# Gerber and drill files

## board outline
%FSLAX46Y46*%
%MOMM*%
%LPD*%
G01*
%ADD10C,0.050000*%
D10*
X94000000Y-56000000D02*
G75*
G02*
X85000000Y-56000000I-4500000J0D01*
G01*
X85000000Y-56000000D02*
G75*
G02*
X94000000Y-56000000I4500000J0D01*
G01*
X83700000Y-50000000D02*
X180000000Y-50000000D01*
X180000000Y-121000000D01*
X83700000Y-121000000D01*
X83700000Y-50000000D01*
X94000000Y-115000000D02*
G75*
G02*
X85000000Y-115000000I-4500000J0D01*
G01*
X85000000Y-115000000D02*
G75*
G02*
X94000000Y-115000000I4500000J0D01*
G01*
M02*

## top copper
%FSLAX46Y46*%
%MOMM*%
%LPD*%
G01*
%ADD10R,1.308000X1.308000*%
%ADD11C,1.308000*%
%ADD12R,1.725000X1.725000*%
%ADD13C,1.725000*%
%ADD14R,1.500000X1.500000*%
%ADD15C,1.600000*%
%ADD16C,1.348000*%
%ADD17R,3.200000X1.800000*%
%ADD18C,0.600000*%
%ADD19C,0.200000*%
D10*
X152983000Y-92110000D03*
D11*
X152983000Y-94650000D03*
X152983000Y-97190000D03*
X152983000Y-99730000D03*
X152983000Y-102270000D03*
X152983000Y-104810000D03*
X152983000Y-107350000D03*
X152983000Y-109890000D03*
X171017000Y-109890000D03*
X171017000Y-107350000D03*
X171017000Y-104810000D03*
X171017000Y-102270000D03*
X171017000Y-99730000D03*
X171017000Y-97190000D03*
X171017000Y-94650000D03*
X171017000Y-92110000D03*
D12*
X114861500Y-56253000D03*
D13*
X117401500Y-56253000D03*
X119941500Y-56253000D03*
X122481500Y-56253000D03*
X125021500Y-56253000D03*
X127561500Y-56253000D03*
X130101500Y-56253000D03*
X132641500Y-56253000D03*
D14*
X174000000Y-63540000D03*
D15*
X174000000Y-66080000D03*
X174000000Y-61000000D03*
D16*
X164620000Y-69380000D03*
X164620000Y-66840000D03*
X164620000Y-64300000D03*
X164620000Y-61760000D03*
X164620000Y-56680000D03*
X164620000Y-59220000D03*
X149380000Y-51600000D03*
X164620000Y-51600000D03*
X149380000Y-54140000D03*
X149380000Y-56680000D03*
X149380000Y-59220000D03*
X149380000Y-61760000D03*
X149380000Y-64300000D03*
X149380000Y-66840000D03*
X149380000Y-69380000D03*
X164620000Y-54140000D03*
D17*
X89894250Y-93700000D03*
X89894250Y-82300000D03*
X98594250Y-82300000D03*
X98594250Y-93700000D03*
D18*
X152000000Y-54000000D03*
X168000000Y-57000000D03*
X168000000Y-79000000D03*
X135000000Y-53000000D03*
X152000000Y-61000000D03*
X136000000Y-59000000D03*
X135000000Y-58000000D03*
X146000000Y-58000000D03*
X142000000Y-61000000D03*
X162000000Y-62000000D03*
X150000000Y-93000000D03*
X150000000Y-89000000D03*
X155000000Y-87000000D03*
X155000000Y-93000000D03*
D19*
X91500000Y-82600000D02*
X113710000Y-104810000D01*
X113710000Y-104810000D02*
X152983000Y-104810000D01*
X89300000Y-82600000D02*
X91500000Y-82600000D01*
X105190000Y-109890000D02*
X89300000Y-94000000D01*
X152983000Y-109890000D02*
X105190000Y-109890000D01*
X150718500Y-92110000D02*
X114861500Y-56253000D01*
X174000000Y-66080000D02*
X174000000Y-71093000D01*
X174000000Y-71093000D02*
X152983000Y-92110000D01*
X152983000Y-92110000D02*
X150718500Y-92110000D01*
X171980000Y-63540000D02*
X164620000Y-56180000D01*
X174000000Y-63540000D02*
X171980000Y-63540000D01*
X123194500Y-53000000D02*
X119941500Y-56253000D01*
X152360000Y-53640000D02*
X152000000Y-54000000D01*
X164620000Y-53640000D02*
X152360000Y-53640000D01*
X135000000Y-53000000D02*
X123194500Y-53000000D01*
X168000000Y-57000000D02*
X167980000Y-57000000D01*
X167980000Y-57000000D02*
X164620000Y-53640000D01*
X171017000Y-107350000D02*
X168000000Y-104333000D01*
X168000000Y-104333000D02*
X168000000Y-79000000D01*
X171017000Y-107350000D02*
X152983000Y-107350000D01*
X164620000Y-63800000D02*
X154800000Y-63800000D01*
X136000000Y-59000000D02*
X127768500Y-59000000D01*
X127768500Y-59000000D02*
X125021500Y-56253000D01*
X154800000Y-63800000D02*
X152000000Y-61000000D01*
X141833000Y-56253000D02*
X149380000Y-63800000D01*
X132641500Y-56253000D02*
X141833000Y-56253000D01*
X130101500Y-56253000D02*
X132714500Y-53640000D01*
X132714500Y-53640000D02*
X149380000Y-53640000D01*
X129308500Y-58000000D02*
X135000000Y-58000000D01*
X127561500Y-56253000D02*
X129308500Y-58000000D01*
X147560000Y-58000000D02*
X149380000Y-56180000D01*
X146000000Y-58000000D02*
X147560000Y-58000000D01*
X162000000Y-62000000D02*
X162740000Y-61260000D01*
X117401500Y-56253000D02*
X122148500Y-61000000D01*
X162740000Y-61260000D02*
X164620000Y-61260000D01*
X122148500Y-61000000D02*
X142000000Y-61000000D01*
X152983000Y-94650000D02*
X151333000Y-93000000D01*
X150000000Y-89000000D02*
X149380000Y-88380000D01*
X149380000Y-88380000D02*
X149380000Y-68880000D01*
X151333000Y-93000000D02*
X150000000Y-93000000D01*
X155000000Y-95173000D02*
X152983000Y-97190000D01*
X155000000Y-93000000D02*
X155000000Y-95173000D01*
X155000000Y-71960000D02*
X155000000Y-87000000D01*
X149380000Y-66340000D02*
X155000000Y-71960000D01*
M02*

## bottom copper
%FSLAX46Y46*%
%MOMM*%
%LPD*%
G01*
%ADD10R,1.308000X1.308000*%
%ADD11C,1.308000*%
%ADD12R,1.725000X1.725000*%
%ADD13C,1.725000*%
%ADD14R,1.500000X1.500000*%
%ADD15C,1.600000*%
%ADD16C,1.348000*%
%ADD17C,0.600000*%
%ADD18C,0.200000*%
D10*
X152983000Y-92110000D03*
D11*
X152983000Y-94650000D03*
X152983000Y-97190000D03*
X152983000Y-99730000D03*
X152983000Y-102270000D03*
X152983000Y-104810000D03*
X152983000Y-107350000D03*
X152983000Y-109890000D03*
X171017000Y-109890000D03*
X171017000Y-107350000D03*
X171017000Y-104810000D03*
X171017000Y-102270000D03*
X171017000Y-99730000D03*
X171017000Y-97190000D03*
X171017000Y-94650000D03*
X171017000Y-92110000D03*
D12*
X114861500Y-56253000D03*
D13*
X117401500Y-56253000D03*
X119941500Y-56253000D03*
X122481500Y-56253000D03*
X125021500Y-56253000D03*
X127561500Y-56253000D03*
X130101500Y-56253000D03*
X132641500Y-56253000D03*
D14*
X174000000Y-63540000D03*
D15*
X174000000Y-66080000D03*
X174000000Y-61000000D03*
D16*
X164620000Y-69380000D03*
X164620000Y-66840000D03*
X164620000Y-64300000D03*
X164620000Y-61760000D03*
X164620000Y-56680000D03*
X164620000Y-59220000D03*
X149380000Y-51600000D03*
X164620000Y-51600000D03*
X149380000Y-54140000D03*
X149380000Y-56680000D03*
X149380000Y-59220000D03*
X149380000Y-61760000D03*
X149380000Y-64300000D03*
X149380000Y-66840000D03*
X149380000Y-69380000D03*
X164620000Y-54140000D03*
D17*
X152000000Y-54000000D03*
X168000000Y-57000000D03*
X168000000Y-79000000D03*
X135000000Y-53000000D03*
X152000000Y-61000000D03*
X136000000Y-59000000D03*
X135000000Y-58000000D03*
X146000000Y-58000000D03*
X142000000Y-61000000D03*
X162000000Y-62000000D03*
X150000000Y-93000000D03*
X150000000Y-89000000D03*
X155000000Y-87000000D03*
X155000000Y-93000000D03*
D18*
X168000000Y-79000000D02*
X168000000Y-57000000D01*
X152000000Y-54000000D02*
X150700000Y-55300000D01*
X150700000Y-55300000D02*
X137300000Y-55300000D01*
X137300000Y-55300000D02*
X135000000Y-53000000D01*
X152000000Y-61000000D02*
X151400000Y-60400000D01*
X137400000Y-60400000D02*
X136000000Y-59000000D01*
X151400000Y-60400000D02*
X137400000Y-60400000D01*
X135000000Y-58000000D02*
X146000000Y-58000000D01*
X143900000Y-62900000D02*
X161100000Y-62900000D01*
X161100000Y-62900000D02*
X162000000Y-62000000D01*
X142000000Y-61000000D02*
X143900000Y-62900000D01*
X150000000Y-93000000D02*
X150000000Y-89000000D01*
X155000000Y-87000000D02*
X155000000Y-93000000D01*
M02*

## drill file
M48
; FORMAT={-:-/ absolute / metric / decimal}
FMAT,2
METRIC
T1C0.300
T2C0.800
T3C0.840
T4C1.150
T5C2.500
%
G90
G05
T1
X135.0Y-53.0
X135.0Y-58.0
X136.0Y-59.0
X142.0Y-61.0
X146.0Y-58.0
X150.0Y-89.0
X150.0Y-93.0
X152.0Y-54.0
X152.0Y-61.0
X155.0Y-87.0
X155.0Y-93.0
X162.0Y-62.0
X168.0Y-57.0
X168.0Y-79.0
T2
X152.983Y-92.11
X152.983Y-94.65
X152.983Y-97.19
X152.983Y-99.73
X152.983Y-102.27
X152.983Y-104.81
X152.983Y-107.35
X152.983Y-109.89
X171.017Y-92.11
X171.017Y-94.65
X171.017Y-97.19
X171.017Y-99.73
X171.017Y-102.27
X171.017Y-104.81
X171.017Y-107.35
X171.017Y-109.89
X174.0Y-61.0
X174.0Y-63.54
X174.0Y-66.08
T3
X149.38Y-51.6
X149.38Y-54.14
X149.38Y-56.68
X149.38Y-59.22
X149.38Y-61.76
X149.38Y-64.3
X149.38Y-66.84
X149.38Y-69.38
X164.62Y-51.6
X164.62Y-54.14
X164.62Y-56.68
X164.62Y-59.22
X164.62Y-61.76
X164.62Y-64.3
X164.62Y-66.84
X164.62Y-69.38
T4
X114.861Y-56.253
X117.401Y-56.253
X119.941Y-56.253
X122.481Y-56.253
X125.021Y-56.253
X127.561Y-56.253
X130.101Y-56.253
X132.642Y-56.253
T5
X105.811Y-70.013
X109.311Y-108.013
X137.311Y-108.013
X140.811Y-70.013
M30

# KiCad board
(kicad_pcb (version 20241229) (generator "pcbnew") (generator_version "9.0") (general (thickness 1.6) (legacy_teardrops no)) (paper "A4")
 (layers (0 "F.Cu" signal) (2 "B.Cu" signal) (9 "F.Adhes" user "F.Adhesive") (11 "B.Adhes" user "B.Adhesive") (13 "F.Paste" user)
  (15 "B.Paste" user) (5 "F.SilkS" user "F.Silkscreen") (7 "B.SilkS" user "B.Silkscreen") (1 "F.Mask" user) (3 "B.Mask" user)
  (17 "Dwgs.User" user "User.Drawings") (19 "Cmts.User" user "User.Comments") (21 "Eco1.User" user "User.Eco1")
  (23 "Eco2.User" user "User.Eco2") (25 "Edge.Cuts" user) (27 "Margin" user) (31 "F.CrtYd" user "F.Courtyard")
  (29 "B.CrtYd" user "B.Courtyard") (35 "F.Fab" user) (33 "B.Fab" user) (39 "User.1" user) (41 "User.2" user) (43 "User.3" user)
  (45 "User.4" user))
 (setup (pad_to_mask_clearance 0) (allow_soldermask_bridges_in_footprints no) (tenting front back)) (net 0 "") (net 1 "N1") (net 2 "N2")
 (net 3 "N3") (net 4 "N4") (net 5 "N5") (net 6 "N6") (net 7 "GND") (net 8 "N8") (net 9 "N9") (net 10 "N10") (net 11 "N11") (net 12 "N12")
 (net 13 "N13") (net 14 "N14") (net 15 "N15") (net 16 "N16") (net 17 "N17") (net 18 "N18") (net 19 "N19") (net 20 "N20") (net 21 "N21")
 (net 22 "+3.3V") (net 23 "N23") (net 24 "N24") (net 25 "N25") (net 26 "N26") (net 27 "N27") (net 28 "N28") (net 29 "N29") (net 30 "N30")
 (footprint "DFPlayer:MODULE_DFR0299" (layer "F.Cu") (at 162 101)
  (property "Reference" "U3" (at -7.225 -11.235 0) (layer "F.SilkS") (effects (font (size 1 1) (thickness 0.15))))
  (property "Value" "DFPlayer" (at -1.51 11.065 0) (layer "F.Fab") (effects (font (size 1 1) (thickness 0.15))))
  (pad "1" thru_hole rect (at -9.017 -8.89) (size 1.308 1.308) (drill 0.8) (layers "*.Cu" "*.Mask") (remove_unused_layers no) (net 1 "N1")
   (solder_mask_margin 0.102))
  (pad "2" thru_hole circle (at -9.017 -6.35) (size 1.308 1.308) (drill 0.8) (layers "*.Cu" "*.Mask") (remove_unused_layers no) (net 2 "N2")
   (solder_mask_margin 0.102))
  (pad "3" thru_hole circle (at -9.017 -3.81) (size 1.308 1.308) (drill 0.8) (layers "*.Cu" "*.Mask") (remove_unused_layers no) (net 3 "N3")
   (solder_mask_margin 0.102))
  (pad "4" thru_hole circle (at -9.017 -1.27) (size 1.308 1.308) (drill 0.8) (layers "*.Cu" "*.Mask") (remove_unused_layers no) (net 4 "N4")
   (solder_mask_margin 0.102))
  (pad "5" thru_hole circle (at -9.017 1.27) (size 1.308 1.308) (drill 0.8) (layers "*.Cu" "*.Mask") (remove_unused_layers no) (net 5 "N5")
   (solder_mask_margin 0.102))
  (pad "6" thru_hole circle (at -9.017 3.81) (size 1.308 1.308) (drill 0.8) (layers "*.Cu" "*.Mask") (remove_unused_layers no) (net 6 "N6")
   (solder_mask_margin 0.102))
  (pad "7" thru_hole circle (at -9.017 6.35) (size 1.308 1.308) (drill 0.8) (layers "*.Cu" "*.Mask") (remove_unused_layers no) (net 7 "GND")
   (solder_mask_margin 0.102))
  (pad "8" thru_hole circle (at -9.017 8.89) (size 1.308 1.308) (drill 0.8) (layers "*.Cu" "*.Mask") (remove_unused_layers no) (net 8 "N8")
   (solder_mask_margin 0.102))
  (pad "9" thru_hole circle (at 9.017 8.89) (size 1.308 1.308) (drill 0.8) (layers "*.Cu" "*.Mask") (remove_unused_layers no) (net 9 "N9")
   (solder_mask_margin 0.102))
  (pad "10" thru_hole circle (at 9.017 6.35) (size 1.308 1.308) (drill 0.8) (layers "*.Cu" "*.Mask") (remove_unused_layers no) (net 7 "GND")
   (solder_mask_margin 0.102))
  (pad "11" thru_hole circle (at 9.017 3.81) (size 1.308 1.308) (drill 0.8) (layers "*.Cu" "*.Mask") (remove_unused_layers no)
   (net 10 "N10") (solder_mask_margin 0.102))
  (pad "12" thru_hole circle (at 9.017 1.27) (size 1.308 1.308) (drill 0.8) (layers "*.Cu" "*.Mask") (remove_unused_layers no)
   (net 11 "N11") (solder_mask_margin 0.102))
  (pad "13" thru_hole circle (at 9.017 -1.27) (size 1.308 1.308) (drill 0.8) (layers "*.Cu" "*.Mask") (remove_unused_layers no)
   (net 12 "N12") (solder_mask_margin 0.102))
  (pad "14" thru_hole circle (at 9.017 -3.81) (size 1.308 1.308) (drill 0.8) (layers "*.Cu" "*.Mask") (remove_unused_layers no)
   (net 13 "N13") (solder_mask_margin 0.102))
  (pad "15" thru_hole circle (at 9.017 -6.35) (size 1.308 1.308) (drill 0.8) (layers "*.Cu" "*.Mask") (remove_unused_layers no)
   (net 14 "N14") (solder_mask_margin 0.102))
  (pad "16" thru_hole circle (at 9.017 -8.89) (size 1.308 1.308) (drill 0.8) (layers "*.Cu" "*.Mask") (remove_unused_layers no)
   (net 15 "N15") (solder_mask_margin 0.102)))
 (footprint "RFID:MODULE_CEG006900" (layer "F.Cu") (at 123.3115 84.013)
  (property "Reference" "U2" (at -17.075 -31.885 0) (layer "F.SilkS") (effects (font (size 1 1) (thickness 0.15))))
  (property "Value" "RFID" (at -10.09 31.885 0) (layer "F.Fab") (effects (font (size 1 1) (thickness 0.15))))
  (pad "" np_thru_hole circle (at -17.5 -14) (size 2.5 2.5) (drill 2.5) (layers "*.Cu" "*.Mask"))
  (pad "" np_thru_hole circle (at -14 24) (size 2.5 2.5) (drill 2.5) (layers "*.Cu" "*.Mask"))
  (pad "" np_thru_hole circle (at 14 24) (size 2.5 2.5) (drill 2.5) (layers "*.Cu" "*.Mask"))
  (pad "" np_thru_hole circle (at 17.5 -14) (size 2.5 2.5) (drill 2.5) (layers "*.Cu" "*.Mask"))
  (pad "1" thru_hole rect (at -8.45 -27.76) (size 1.725 1.725) (drill 1.15) (layers "*.Cu" "*.Mask") (remove_unused_layers no) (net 1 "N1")
   (solder_mask_margin 0.102))
  (pad "2" thru_hole circle (at -5.91 -27.76) (size 1.725 1.725) (drill 1.15) (layers "*.Cu" "*.Mask") (remove_unused_layers no)
   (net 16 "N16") (solder_mask_margin 0.102))
  (pad "3" thru_hole circle (at -3.37 -27.76) (size 1.725 1.725) (drill 1.15) (layers "*.Cu" "*.Mask") (remove_unused_layers no)
   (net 7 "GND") (solder_mask_margin 0.102))
  (pad "4" thru_hole circle (at -0.83 -27.76) (size 1.725 1.725) (drill 1.15) (layers "*.Cu" "*.Mask") (remove_unused_layers no)
   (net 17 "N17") (solder_mask_margin 0.102))
  (pad "5" thru_hole circle (at 1.71 -27.76) (size 1.725 1.725) (drill 1.15) (layers "*.Cu" "*.Mask") (remove_unused_layers no)
   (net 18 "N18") (solder_mask_margin 0.102))
  (pad "6" thru_hole circle (at 4.25 -27.76) (size 1.725 1.725) (drill 1.15) (layers "*.Cu" "*.Mask") (remove_unused_layers no)
   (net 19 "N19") (solder_mask_margin 0.102))
  (pad "7" thru_hole circle (at 6.79 -27.76) (size 1.725 1.725) (drill 1.15) (layers "*.Cu" "*.Mask") (remove_unused_layers no)
   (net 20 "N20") (solder_mask_margin 0.102))
  (pad "8" thru_hole circle (at 9.33 -27.76) (size 1.725 1.725) (drill 1.15) (layers "*.Cu" "*.Mask") (remove_unused_layers no)
   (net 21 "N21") (solder_mask_margin 0.102)))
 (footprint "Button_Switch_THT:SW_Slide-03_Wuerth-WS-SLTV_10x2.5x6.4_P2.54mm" (layer "F.Cu") (at 174 63.54 90)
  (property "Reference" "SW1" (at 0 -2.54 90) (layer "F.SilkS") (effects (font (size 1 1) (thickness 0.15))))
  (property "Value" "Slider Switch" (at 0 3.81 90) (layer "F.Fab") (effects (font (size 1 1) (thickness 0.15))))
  (pad "1" thru_hole rect (at 0 0 90) (size 1.5 1.5) (drill 0.8) (layers "*.Cu" "*.Mask") (remove_unused_layers no) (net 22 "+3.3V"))
  (pad "2" thru_hole circle (at -2.54 0 90) (size 1.6 1.6) (drill 0.8) (layers "*.Cu" "*.Mask") (remove_unused_layers no) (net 1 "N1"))
  (pad "3" thru_hole circle (at 2.54 0 90) (size 1.6 1.6) (drill 0.8) (layers "*.Cu" "*.Mask") (remove_unused_layers no) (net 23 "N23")))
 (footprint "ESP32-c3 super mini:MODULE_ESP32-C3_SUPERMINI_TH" (layer "F.Cu") (at 157 61.5)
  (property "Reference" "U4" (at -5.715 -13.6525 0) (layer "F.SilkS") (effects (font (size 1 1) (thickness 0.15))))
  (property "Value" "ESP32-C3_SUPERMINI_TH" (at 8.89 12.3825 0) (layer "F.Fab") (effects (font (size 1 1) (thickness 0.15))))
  (pad "0" thru_hole circle (at 7.62 7.88) (size 1.348 1.348) (drill 0.84) (layers "*.Cu" "*.Mask") (remove_unused_layers no) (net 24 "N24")
   (solder_mask_margin 0.102))
  (pad "1" thru_hole circle (at 7.62 5.34) (size 1.348 1.348) (drill 0.84) (layers "*.Cu" "*.Mask") (remove_unused_layers no) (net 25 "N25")
   (solder_mask_margin 0.102))
  (pad "2" thru_hole circle (at 7.62 2.8) (size 1.348 1.348) (drill 0.84) (layers "*.Cu" "*.Mask") (remove_unused_layers no) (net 18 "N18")
   (solder_mask_margin 0.102))
  (pad "3" thru_hole circle (at 7.62 0.26) (size 1.348 1.348) (drill 0.84) (layers "*.Cu" "*.Mask") (remove_unused_layers no) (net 16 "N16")
   (solder_mask_margin 0.102))
  (pad "3.3" thru_hole circle (at 7.62 -4.82) (size 1.348 1.348) (drill 0.84) (layers "*.Cu" "*.Mask") (remove_unused_layers no)
   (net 22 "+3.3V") (solder_mask_margin 0.102))
  (pad "4" thru_hole circle (at 7.62 -2.28) (size 1.348 1.348) (drill 0.84) (layers "*.Cu" "*.Mask") (remove_unused_layers no)
   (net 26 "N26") (solder_mask_margin 0.102))
  (pad "5" thru_hole circle (at -7.62 -9.9) (size 1.348 1.348) (drill 0.84) (layers "*.Cu" "*.Mask") (remove_unused_layers no)
   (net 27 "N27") (solder_mask_margin 0.102))
  (pad "5V" thru_hole circle (at 7.62 -9.9) (size 1.348 1.348) (drill 0.84) (layers "*.Cu" "*.Mask") (remove_unused_layers no)
   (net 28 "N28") (solder_mask_margin 0.102))
  (pad "6" thru_hole circle (at -7.62 -7.36) (size 1.348 1.348) (drill 0.84) (layers "*.Cu" "*.Mask") (remove_unused_layers no)
   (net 20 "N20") (solder_mask_margin 0.102))
  (pad "7" thru_hole circle (at -7.62 -4.82) (size 1.348 1.348) (drill 0.84) (layers "*.Cu" "*.Mask") (remove_unused_layers no)
   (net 19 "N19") (solder_mask_margin 0.102))
  (pad "8" thru_hole circle (at -7.62 -2.28) (size 1.348 1.348) (drill 0.84) (layers "*.Cu" "*.Mask") (remove_unused_layers no)
   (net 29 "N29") (solder_mask_margin 0.102))
  (pad "9" thru_hole circle (at -7.62 0.26) (size 1.348 1.348) (drill 0.84) (layers "*.Cu" "*.Mask") (remove_unused_layers no)
   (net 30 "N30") (solder_mask_margin 0.102))
  (pad "10" thru_hole circle (at -7.62 2.8) (size 1.348 1.348) (drill 0.84) (layers "*.Cu" "*.Mask") (remove_unused_layers no)
   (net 21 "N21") (solder_mask_margin 0.102))
  (pad "20" thru_hole circle (at -7.62 5.34) (size 1.348 1.348) (drill 0.84) (layers "*.Cu" "*.Mask") (remove_unused_layers no) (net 3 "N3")
   (solder_mask_margin 0.102))
  (pad "21" thru_hole circle (at -7.62 7.88) (size 1.348 1.348) (drill 0.84) (layers "*.Cu" "*.Mask") (remove_unused_layers no) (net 2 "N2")
   (solder_mask_margin 0.102))
  (pad "G" thru_hole circle (at 7.62 -7.36) (size 1.348 1.348) (drill 0.84) (layers "*.Cu" "*.Mask") (remove_unused_layers no) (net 7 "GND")
   (solder_mask_margin 0.102)))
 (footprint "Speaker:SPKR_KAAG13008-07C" (layer "F.Cu") (at 94.24425 88)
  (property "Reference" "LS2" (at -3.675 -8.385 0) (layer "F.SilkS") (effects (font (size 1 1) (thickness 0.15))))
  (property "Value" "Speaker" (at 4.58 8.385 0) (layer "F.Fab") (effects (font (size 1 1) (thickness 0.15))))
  (pad "N" smd rect (at -4.35 5.7) (size 3.2 1.8) (layers "F.Cu" "F.Mask" "F.Paste") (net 8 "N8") (solder_mask_margin 0.102))
  (pad "P" smd rect (at -4.35 -5.7) (size 3.2 1.8) (layers "F.Cu" "F.Mask" "F.Paste") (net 6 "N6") (solder_mask_margin 0.102))
  (pad "S1" smd rect (at 4.35 -5.7) (size 3.2 1.8) (layers "F.Cu" "F.Mask" "F.Paste") (solder_mask_margin 0.102))
  (pad "S2" smd rect (at 4.35 5.7) (size 3.2 1.8) (layers "F.Cu" "F.Mask" "F.Paste") (solder_mask_margin 0.102)))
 (gr_circle (center 89.5 56) (end 89.5 51.5) (stroke (width 0.05) (type default)) (fill no) (layer "Edge.Cuts"))
 (gr_rect (start 83.7 50) (end 180 121) (stroke (width 0.05) (type default)) (fill no) (layer "Edge.Cuts"))
 (gr_circle (center 89.5 115) (end 89.5 110.5) (stroke (width 0.05) (type default)) (fill no) (layer "Edge.Cuts"))
 (segment (start 91.5 82.6) (end 113.71 104.81) (width 0.2) (layer "F.Cu") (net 6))
 (segment (start 113.71 104.81) (end 152.983 104.81) (width 0.2) (layer "F.Cu") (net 6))
 (segment (start 89.3 82.6) (end 91.5 82.6) (width 0.2) (layer "F.Cu") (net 6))
 (segment (start 105.19 109.89) (end 89.3 94) (width 0.2) (layer "F.Cu") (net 8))
 (segment (start 152.983 109.89) (end 105.19 109.89) (width 0.2) (layer "F.Cu") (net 8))
 (segment (start 150.7185 92.11) (end 114.8615 56.253) (width 0.2) (layer "F.Cu") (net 1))
 (segment (start 174 66.08) (end 174 71.093) (width 0.2) (layer "F.Cu") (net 1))
 (segment (start 174 71.093) (end 152.983 92.11) (width 0.2) (layer "F.Cu") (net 1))
 (segment (start 152.983 92.11) (end 150.7185 92.11) (width 0.2) (layer "F.Cu") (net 1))
 (segment (start 171.98 63.54) (end 164.62 56.18) (width 0.2) (layer "F.Cu") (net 22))
 (segment (start 174 63.54) (end 171.98 63.54) (width 0.2) (layer "F.Cu") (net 22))
 (segment (start 123.1945 53) (end 119.9415 56.253) (width 0.2) (layer "F.Cu") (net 7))
 (segment (start 152.36 53.64) (end 152 54) (width 0.2) (layer "F.Cu") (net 7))
 (segment (start 164.62 53.64) (end 152.36 53.64) (width 0.2) (layer "F.Cu") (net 7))
 (segment (start 135 53) (end 123.1945 53) (width 0.2) (layer "F.Cu") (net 7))
 (segment (start 168 57) (end 167.98 57) (width 0.2) (layer "F.Cu") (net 7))
 (segment (start 167.98 57) (end 164.62 53.64) (width 0.2) (layer "F.Cu") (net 7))
 (segment (start 171.017 107.35) (end 168 104.333) (width 0.2) (layer "F.Cu") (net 7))
 (segment (start 168 104.333) (end 168 79) (width 0.2) (layer "F.Cu") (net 7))
 (segment (start 171.017 107.35) (end 152.983 107.35) (width 0.2) (layer "F.Cu") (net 7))
 (via (at 152 54) (size 0.6) (drill 0.3) (layers "F.Cu" "B.Cu") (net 7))
 (via (at 168 57) (size 0.6) (drill 0.3) (layers "F.Cu" "B.Cu") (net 7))
 (via (at 168 79) (size 0.6) (drill 0.3) (layers "F.Cu" "B.Cu") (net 7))
 (via (at 135 53) (size 0.6) (drill 0.3) (layers "F.Cu" "B.Cu") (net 7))
 (segment (start 168 79) (end 168 57) (width 0.2) (layer "B.Cu") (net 7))
 (segment (start 152 54) (end 150.7 55.3) (width 0.2) (layer "B.Cu") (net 7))
 (segment (start 150.7 55.3) (end 137.3 55.3) (width 0.2) (layer "B.Cu") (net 7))
 (segment (start 137.3 55.3) (end 135 53) (width 0.2) (layer "B.Cu") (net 7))
 (segment (start 164.62 63.8) (end 154.8 63.8) (width 0.2) (layer "F.Cu") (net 18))
 (segment (start 136 59) (end 127.7685 59) (width 0.2) (layer "F.Cu") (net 18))
 (segment (start 127.7685 59) (end 125.0215 56.253) (width 0.2) (layer "F.Cu") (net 18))
 (segment (start 154.8 63.8) (end 152 61) (width 0.2) (layer "F.Cu") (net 18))
 (via (at 152 61) (size 0.6) (drill 0.3) (layers "F.Cu" "B.Cu") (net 18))
 (via (at 136 59) (size 0.6) (drill 0.3) (layers "F.Cu" "B.Cu") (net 18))
 (segment (start 152 61) (end 151.4 60.4) (width 0.2) (layer "B.Cu") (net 18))
 (segment (start 137.4 60.4) (end 136 59) (width 0.2) (layer "B.Cu") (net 18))
 (segment (start 151.4 60.4) (end 137.4 60.4) (width 0.2) (layer "B.Cu") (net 18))
 (segment (start 141.833 56.253) (end 149.38 63.8) (width 0.2) (layer "F.Cu") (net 21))
 (segment (start 132.6415 56.253) (end 141.833 56.253) (width 0.2) (layer "F.Cu") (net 21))
 (segment (start 130.1015 56.253) (end 132.7145 53.64) (width 0.2) (layer "F.Cu") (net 20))
 (segment (start 132.7145 53.64) (end 149.38 53.64) (width 0.2) (layer "F.Cu") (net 20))
 (segment (start 129.3085 58) (end 135 58) (width 0.2) (layer "F.Cu") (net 19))
 (segment (start 127.5615 56.253) (end 129.3085 58) (width 0.2) (layer "F.Cu") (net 19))
 (segment (start 147.56 58) (end 149.38 56.18) (width 0.2) (layer "F.Cu") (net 19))
 (segment (start 146 58) (end 147.56 58) (width 0.2) (layer "F.Cu") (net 19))
 (via (at 135 58) (size 0.6) (drill 0.3) (layers "F.Cu" "B.Cu") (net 19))
 (via (at 146 58) (size 0.6) (drill 0.3) (layers "F.Cu" "B.Cu") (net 19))
 (segment (start 135 58) (end 146 58) (width 0.2) (layer "B.Cu") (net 19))
 (segment (start 162 62) (end 162.74 61.26) (width 0.2) (layer "F.Cu") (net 16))
 (segment (start 117.4015 56.253) (end 122.1485 61) (width 0.2) (layer "F.Cu") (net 16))
 (segment (start 162.74 61.26) (end 164.62 61.26) (width 0.2) (layer "F.Cu") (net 16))
 (segment (start 122.1485 61) (end 142 61) (width 0.2) (layer "F.Cu") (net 16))
 (via (at 142 61) (size 0.6) (drill 0.3) (layers "F.Cu" "B.Cu") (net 16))
 (via (at 162 62) (size 0.6) (drill 0.3) (layers "F.Cu" "B.Cu") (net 16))
 (segment (start 143.9 62.9) (end 161.1 62.9) (width 0.2) (layer "B.Cu") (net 16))
 (segment (start 161.1 62.9) (end 162 62) (width 0.2) (layer "B.Cu") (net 16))
 (segment (start 142 61) (end 143.9 62.9) (width 0.2) (layer "B.Cu") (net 16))
 (segment (start 152.983 94.65) (end 151.333 93) (width 0.2) (layer "F.Cu") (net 2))
 (segment (start 150 89) (end 149.38 88.38) (width 0.2) (layer "F.Cu") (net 2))
 (segment (start 149.38 88.38) (end 149.38 68.88) (width 0.2) (layer "F.Cu") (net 2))
 (segment (start 151.333 93) (end 150 93) (width 0.2) (layer "F.Cu") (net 2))
 (via (at 150 93) (size 0.6) (drill 0.3) (layers "F.Cu" "B.Cu") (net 2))
 (via (at 150 89) (size 0.6) (drill 0.3) (layers "F.Cu" "B.Cu") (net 2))
 (segment (start 150 93) (end 150 89) (width 0.2) (layer "B.Cu") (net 2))
 (segment (start 155 95.173) (end 152.983 97.19) (width 0.2) (layer "F.Cu") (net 3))
 (segment (start 155 93) (end 155 95.173) (width 0.2) (layer "F.Cu") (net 3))
 (segment (start 155 71.96) (end 155 87) (width 0.2) (layer "F.Cu") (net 3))
 (segment (start 149.38 66.34) (end 155 71.96) (width 0.2) (layer "F.Cu") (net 3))
 (via (at 155 87) (size 0.6) (drill 0.3) (layers "F.Cu" "B.Cu") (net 3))
 (via (at 155 93) (size 0.6) (drill 0.3) (layers "F.Cu" "B.Cu") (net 3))
 (segment (start 155 87) (end 155 93) (width 0.2) (layer "B.Cu") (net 3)))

